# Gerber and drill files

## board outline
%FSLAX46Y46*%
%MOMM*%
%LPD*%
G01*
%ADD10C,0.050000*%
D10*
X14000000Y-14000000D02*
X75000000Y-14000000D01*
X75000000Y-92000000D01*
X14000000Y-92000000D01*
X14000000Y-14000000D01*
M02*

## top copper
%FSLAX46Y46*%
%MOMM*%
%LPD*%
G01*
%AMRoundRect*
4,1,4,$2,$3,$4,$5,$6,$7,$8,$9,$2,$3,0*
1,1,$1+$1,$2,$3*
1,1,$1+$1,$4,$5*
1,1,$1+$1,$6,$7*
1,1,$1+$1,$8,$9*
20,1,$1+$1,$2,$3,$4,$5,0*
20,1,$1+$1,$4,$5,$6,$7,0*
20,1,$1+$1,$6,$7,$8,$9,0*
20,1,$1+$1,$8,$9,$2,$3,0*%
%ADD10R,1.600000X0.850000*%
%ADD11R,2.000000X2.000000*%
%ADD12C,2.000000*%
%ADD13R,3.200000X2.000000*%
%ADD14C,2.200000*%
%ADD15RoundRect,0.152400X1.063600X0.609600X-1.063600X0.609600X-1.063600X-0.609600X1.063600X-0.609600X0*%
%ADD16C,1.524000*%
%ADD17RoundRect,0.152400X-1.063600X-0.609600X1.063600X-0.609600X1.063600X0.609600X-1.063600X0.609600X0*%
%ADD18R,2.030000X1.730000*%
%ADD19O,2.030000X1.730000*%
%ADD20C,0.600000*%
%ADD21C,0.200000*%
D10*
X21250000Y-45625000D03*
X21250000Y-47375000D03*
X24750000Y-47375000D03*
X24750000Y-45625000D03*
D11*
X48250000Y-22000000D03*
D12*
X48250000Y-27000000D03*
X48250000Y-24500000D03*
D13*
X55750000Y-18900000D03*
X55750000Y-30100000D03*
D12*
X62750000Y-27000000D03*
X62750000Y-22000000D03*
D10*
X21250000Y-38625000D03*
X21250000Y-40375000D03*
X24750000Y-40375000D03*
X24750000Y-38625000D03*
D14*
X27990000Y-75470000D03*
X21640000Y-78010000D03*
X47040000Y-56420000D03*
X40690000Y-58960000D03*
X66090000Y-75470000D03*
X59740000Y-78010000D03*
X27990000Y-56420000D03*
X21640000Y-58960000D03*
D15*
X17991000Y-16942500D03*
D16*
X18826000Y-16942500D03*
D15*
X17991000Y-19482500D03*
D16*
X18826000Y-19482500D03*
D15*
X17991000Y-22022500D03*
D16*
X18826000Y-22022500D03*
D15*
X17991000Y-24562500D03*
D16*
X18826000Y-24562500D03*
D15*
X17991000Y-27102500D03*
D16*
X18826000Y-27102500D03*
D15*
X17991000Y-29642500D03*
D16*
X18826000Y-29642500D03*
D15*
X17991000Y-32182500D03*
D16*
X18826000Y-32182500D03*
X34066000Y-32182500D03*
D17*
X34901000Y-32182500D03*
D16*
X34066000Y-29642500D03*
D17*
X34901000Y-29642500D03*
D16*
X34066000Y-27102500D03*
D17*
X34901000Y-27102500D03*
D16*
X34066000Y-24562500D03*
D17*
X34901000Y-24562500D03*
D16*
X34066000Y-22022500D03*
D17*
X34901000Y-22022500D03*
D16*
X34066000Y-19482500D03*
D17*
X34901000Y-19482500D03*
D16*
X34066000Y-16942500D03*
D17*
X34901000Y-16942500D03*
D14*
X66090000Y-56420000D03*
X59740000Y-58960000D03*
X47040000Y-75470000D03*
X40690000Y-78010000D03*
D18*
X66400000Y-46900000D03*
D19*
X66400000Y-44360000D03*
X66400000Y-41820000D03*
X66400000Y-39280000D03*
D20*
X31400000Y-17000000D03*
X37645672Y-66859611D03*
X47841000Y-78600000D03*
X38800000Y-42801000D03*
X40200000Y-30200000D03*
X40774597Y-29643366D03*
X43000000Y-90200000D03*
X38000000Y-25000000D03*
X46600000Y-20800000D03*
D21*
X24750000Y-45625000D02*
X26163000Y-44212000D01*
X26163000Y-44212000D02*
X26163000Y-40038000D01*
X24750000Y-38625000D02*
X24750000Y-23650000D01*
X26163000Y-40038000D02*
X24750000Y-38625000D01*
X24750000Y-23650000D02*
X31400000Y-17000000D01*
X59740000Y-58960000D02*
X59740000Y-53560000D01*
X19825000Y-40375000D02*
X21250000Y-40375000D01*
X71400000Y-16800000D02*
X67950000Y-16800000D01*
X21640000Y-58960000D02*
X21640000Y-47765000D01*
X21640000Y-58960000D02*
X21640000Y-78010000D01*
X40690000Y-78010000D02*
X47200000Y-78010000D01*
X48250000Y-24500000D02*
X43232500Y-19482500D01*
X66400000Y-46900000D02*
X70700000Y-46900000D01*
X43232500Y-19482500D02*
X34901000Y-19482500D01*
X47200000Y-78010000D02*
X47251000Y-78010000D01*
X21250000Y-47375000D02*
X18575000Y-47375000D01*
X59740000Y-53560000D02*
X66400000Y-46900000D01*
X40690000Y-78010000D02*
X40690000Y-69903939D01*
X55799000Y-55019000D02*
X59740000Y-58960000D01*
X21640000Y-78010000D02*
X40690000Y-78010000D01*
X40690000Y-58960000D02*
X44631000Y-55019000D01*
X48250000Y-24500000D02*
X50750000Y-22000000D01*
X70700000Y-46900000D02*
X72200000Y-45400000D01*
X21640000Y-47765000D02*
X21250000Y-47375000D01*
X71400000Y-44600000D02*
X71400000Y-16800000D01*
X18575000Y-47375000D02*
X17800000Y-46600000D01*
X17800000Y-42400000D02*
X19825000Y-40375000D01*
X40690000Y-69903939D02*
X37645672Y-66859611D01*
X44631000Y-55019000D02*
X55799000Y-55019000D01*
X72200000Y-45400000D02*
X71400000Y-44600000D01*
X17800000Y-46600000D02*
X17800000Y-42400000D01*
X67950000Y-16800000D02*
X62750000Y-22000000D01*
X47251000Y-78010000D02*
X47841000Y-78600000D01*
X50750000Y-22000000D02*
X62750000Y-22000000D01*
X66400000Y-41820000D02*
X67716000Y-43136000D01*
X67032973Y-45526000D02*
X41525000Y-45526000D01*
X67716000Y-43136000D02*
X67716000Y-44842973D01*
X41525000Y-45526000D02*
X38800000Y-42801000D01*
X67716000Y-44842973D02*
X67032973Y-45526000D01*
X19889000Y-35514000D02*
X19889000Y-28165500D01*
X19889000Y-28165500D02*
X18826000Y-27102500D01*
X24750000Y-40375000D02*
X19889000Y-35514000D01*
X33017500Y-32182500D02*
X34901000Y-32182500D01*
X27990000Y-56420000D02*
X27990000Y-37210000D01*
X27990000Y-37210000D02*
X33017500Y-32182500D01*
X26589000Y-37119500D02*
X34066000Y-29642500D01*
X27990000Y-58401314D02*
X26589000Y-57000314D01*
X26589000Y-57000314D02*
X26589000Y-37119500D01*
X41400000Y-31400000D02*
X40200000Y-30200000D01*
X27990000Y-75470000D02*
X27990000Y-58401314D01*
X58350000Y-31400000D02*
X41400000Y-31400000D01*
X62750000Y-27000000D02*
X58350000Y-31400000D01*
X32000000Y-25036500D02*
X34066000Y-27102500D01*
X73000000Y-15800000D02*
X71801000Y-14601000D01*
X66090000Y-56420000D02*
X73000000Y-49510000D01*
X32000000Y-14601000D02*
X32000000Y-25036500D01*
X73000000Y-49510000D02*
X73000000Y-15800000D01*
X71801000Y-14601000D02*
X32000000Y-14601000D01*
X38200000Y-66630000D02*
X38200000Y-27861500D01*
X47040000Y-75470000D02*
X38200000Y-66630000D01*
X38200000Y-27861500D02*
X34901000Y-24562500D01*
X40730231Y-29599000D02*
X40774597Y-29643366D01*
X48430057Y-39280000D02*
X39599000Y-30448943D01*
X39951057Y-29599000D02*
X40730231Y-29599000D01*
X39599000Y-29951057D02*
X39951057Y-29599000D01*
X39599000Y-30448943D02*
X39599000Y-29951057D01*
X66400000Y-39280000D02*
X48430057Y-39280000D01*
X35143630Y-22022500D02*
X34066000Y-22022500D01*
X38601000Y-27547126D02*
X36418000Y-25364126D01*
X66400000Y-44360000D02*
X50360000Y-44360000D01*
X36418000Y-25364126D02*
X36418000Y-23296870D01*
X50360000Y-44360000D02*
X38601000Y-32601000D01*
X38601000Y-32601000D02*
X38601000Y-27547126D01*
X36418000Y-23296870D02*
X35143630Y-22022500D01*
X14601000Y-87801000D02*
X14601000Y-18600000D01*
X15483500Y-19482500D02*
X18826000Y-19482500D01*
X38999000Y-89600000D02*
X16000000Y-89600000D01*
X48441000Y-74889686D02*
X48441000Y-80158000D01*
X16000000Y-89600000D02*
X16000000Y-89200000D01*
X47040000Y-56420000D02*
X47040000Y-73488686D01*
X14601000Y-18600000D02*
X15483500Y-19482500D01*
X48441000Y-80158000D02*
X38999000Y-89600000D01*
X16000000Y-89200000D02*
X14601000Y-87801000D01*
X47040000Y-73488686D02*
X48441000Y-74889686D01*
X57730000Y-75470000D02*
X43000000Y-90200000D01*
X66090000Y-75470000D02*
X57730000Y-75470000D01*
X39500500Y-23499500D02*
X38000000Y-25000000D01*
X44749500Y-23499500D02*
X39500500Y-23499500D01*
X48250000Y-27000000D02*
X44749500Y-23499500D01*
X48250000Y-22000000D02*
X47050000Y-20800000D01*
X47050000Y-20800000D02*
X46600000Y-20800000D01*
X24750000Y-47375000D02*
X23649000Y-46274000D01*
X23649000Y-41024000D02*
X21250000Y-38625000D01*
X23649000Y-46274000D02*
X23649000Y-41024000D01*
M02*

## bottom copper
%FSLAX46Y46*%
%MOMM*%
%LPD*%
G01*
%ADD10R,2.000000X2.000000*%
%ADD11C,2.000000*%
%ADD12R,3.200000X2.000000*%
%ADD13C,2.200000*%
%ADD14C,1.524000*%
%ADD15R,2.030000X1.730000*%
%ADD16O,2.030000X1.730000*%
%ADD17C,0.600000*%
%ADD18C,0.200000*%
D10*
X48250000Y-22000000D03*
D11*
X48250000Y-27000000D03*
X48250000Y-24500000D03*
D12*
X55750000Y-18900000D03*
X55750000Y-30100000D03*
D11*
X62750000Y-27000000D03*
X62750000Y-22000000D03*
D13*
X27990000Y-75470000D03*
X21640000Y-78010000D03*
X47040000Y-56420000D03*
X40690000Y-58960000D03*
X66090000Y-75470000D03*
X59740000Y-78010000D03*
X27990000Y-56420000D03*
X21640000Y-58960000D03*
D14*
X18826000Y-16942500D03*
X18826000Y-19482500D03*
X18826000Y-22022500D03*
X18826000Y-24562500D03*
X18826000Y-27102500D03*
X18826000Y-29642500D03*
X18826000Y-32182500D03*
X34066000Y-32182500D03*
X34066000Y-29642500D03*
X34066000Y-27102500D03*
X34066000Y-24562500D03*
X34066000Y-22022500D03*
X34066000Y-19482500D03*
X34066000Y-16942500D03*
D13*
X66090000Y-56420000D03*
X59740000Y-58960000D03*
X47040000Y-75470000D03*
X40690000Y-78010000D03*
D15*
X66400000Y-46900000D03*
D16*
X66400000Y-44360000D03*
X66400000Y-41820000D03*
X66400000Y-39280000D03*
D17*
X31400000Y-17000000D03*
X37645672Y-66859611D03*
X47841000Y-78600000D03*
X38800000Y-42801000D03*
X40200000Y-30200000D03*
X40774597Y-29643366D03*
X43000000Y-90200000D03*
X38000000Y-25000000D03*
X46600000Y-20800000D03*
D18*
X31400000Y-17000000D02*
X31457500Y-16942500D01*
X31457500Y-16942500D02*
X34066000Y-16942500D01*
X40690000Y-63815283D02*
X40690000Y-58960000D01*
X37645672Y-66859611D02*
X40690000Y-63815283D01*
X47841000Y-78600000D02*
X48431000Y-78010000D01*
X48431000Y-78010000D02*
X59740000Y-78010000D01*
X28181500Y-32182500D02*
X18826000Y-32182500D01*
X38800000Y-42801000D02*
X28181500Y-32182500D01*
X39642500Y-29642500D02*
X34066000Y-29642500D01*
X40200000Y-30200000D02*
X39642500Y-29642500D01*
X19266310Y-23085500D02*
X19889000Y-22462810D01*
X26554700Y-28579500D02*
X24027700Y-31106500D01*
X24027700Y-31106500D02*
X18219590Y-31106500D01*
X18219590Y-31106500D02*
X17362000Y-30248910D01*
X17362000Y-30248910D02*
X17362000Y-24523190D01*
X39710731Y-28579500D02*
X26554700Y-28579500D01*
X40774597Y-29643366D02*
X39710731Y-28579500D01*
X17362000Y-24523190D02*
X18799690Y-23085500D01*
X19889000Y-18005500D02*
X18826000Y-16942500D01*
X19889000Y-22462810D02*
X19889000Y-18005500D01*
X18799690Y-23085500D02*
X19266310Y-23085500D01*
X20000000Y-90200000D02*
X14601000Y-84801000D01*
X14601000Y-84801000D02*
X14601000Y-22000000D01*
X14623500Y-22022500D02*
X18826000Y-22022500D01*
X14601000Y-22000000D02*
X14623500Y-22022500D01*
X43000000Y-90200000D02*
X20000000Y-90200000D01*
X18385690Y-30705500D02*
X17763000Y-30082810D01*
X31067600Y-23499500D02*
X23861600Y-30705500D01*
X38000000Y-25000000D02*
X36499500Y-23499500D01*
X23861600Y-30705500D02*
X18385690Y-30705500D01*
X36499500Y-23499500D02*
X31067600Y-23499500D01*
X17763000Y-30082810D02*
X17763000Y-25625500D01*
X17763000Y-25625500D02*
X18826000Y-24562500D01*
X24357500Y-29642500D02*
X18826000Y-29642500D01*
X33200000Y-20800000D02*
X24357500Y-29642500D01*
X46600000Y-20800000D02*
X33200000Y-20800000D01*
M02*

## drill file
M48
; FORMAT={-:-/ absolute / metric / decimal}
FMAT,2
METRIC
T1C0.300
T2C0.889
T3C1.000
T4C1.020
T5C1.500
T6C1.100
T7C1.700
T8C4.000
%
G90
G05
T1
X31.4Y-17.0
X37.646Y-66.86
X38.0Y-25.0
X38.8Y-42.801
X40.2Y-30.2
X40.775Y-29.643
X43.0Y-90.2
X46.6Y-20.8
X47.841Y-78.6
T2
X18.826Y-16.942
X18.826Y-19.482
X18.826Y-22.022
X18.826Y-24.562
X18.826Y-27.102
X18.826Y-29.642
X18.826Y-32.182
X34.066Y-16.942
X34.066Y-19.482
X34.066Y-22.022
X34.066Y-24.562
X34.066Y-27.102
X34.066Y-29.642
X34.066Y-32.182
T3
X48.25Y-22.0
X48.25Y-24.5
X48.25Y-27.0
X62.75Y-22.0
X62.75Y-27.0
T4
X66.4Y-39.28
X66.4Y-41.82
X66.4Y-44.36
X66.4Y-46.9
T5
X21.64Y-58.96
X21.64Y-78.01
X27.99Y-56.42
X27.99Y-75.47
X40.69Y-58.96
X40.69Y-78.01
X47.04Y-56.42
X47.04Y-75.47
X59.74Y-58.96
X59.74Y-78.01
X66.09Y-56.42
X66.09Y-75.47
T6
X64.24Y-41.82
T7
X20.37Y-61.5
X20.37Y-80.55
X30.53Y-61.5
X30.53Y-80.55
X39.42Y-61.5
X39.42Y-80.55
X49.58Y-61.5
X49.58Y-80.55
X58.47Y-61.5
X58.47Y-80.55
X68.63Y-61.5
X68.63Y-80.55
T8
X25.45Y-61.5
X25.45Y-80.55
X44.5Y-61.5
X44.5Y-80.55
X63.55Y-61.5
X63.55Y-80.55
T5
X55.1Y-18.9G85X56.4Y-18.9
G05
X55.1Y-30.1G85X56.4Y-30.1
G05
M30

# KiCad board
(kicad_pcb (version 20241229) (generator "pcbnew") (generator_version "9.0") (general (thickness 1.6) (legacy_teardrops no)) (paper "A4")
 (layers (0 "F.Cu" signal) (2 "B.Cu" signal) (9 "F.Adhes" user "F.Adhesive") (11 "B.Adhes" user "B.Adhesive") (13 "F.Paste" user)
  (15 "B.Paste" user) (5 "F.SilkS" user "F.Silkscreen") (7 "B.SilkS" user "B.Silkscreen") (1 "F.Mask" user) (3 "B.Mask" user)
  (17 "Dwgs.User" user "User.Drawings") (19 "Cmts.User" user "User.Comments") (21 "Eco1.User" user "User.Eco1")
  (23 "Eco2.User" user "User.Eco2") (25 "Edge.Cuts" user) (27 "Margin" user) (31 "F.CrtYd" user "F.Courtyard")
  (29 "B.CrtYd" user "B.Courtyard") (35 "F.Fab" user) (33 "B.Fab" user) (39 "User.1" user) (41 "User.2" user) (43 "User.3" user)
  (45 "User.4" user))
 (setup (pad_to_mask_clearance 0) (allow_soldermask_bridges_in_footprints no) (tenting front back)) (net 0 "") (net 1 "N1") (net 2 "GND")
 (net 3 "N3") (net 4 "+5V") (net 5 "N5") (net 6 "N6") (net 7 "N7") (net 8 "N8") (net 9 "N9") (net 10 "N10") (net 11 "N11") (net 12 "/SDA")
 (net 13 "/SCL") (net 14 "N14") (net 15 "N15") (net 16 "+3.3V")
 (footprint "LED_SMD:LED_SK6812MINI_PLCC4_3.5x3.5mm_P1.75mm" (layer "F.Cu") (at 23 46.5)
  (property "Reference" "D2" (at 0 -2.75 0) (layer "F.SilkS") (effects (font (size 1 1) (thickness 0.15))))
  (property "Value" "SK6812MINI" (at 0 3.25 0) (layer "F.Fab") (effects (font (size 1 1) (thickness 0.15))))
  (pad "1" smd rect (at -1.75 -0.875) (size 1.6 0.85) (layers "F.Cu" "F.Mask" "F.Paste") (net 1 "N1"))
  (pad "2" smd rect (at -1.75 0.875) (size 1.6 0.85) (layers "F.Cu" "F.Mask" "F.Paste") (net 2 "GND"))
  (pad "3" smd rect (at 1.75 0.875) (size 1.6 0.85) (layers "F.Cu" "F.Mask" "F.Paste") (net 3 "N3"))
  (pad "4" smd rect (at 1.75 -0.875) (size 1.6 0.85) (layers "F.Cu" "F.Mask" "F.Paste") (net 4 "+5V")))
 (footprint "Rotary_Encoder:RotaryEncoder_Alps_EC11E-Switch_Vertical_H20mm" (layer "F.Cu") (at 48.25 22)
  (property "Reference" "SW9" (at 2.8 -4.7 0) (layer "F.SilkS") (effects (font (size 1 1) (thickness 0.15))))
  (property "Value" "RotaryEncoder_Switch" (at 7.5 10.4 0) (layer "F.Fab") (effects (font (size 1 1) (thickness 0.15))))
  (pad "A" thru_hole rect (at 0 0) (size 2 2) (drill 1) (layers "*.Cu" "*.Mask") (remove_unused_layers no) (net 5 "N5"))
  (pad "B" thru_hole circle (at 0 5) (size 2 2) (drill 1) (layers "*.Cu" "*.Mask") (remove_unused_layers no) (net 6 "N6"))
  (pad "C" thru_hole circle (at 0 2.5) (size 2 2) (drill 1) (layers "*.Cu" "*.Mask") (remove_unused_layers no) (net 2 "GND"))
  (pad "MP" thru_hole rect (at 7.5 -3.1) (size 3.2 2) (drill oval 2.8 1.5) (layers "*.Cu" "*.Mask") (remove_unused_layers no))
  (pad "MP" thru_hole rect (at 7.5 8.1) (size 3.2 2) (drill oval 2.8 1.5) (layers "*.Cu" "*.Mask") (remove_unused_layers no))
  (pad "S1" thru_hole circle (at 14.5 5) (size 2 2) (drill 1) (layers "*.Cu" "*.Mask") (remove_unused_layers no) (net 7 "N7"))
  (pad "S2" thru_hole circle (at 14.5 0) (size 2 2) (drill 1) (layers "*.Cu" "*.Mask") (remove_unused_layers no) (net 2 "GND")))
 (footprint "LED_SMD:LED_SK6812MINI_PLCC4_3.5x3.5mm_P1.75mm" (layer "F.Cu") (at 23 39.5)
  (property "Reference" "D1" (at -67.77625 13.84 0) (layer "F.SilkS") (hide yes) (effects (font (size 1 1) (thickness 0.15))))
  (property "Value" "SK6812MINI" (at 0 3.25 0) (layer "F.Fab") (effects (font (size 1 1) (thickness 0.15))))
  (pad "1" smd rect (at -1.75 -0.875) (size 1.6 0.85) (layers "F.Cu" "F.Mask" "F.Paste") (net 3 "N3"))
  (pad "2" smd rect (at -1.75 0.875) (size 1.6 0.85) (layers "F.Cu" "F.Mask" "F.Paste") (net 2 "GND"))
  (pad "3" smd rect (at 1.75 0.875) (size 1.6 0.85) (layers "F.Cu" "F.Mask" "F.Paste") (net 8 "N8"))
  (pad "4" smd rect (at 1.75 -0.875) (size 1.6 0.85) (layers "F.Cu" "F.Mask" "F.Paste") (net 4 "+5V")))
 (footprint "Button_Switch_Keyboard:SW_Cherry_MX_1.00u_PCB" (layer "F.Cu") (at 27.99 75.47)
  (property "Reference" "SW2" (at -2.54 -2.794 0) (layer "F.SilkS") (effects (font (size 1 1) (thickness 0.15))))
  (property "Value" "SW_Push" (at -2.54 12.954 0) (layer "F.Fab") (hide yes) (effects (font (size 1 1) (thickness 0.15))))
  (pad "" np_thru_hole circle (at -7.62 5.08) (size 1.7 1.7) (drill 1.7) (layers "*.Cu" "*.Mask"))
  (pad "" np_thru_hole circle (at -2.54 5.08) (size 4 4) (drill 4) (layers "*.Cu" "*.Mask"))
  (pad "" np_thru_hole circle (at 2.54 5.08) (size 1.7 1.7) (drill 1.7) (layers "*.Cu" "*.Mask"))
  (pad "1" thru_hole circle (at 0 0) (size 2.2 2.2) (drill 1.5) (layers "*.Cu" "*.Mask") (remove_unused_layers no) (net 7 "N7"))
  (pad "2" thru_hole circle (at -6.35 2.54) (size 2.2 2.2) (drill 1.5) (layers "*.Cu" "*.Mask") (remove_unused_layers no) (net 2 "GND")))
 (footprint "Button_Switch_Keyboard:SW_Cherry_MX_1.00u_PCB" (layer "F.Cu") (at 47.04 56.42)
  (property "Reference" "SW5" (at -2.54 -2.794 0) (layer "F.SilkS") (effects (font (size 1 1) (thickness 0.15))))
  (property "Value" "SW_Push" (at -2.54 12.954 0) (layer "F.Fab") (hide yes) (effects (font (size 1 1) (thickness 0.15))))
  (pad "" np_thru_hole circle (at -7.62 5.08) (size 1.7 1.7) (drill 1.7) (layers "*.Cu" "*.Mask"))
  (pad "" np_thru_hole circle (at -2.54 5.08) (size 4 4) (drill 4) (layers "*.Cu" "*.Mask"))
  (pad "" np_thru_hole circle (at 2.54 5.08) (size 1.7 1.7) (drill 1.7) (layers "*.Cu" "*.Mask"))
  (pad "1" thru_hole circle (at 0 0) (size 2.2 2.2) (drill 1.5) (layers "*.Cu" "*.Mask") (remove_unused_layers no) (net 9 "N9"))
  (pad "2" thru_hole circle (at -6.35 2.54) (size 2.2 2.2) (drill 1.5) (layers "*.Cu" "*.Mask") (remove_unused_layers no) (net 2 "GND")))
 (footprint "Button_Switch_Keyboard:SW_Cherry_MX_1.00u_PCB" (layer "F.Cu") (at 66.09 75.47)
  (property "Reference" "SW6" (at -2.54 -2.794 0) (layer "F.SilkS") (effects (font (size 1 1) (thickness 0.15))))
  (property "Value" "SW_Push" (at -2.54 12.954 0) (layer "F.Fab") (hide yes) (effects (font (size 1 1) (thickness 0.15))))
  (pad "" np_thru_hole circle (at -7.62 5.08) (size 1.7 1.7) (drill 1.7) (layers "*.Cu" "*.Mask"))
  (pad "" np_thru_hole circle (at -2.54 5.08) (size 4 4) (drill 4) (layers "*.Cu" "*.Mask"))
  (pad "" np_thru_hole circle (at 2.54 5.08) (size 1.7 1.7) (drill 1.7) (layers "*.Cu" "*.Mask"))
  (pad "1" thru_hole circle (at 0 0) (size 2.2 2.2) (drill 1.5) (layers "*.Cu" "*.Mask") (remove_unused_layers no) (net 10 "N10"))
  (pad "2" thru_hole circle (at -6.35 2.54) (size 2.2 2.2) (drill 1.5) (layers "*.Cu" "*.Mask") (remove_unused_layers no) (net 2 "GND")))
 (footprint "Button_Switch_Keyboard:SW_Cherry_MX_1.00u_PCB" (layer "F.Cu") (at 27.99 56.42)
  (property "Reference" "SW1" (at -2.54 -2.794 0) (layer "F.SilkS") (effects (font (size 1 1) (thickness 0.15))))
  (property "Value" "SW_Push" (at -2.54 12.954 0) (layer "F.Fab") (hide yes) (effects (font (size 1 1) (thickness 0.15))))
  (pad "" np_thru_hole circle (at -7.62 5.08) (size 1.7 1.7) (drill 1.7) (layers "*.Cu" "*.Mask"))
  (pad "" np_thru_hole circle (at -2.54 5.08) (size 4 4) (drill 4) (layers "*.Cu" "*.Mask"))
  (pad "" np_thru_hole circle (at 2.54 5.08) (size 1.7 1.7) (drill 1.7) (layers "*.Cu" "*.Mask"))
  (pad "1" thru_hole circle (at 0 0) (size 2.2 2.2) (drill 1.5) (layers "*.Cu" "*.Mask") (remove_unused_layers no) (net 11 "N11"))
  (pad "2" thru_hole circle (at -6.35 2.54) (size 2.2 2.2) (drill 1.5) (layers "*.Cu" "*.Mask") (remove_unused_layers no) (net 2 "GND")))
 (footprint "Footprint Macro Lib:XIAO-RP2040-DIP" (layer "F.Cu") (at 26.446 24.5625)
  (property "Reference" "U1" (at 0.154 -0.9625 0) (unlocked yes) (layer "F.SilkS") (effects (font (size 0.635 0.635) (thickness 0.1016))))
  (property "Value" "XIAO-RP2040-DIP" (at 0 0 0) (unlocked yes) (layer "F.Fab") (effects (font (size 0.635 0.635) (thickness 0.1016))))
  (pad "1" smd roundrect (at -8.455 -7.62 180) (size 2.432 1.524) (layers "F.Cu" "F.Mask") (roundrect_rratio 0.1) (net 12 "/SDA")
   (thermal_bridge_angle 45))
  (pad "1" thru_hole circle (at -7.62 -7.62 180) (size 1.524 1.524) (drill 0.889) (layers "*.Cu" "*.Mask") (remove_unused_layers no)
   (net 12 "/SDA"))
  (pad "2" smd roundrect (at -8.455 -5.08 180) (size 2.432 1.524) (layers "F.Cu" "F.Mask") (roundrect_rratio 0.1) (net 9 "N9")
   (thermal_bridge_angle 45))
  (pad "2" thru_hole circle (at -7.62 -5.08 180) (size 1.524 1.524) (drill 0.889) (layers "*.Cu" "*.Mask") (remove_unused_layers no)
   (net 9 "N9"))
  (pad "3" smd roundrect (at -8.455 -2.54 180) (size 2.432 1.524) (layers "F.Cu" "F.Mask") (roundrect_rratio 0.1) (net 10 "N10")
   (thermal_bridge_angle 45))
  (pad "3" thru_hole circle (at -7.62 -2.54 180) (size 1.524 1.524) (drill 0.889) (layers "*.Cu" "*.Mask") (remove_unused_layers no)
   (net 10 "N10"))
  (pad "4" smd roundrect (at -8.455 0 180) (size 2.432 1.524) (layers "F.Cu" "F.Mask") (roundrect_rratio 0.1) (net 6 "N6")
   (thermal_bridge_angle 45))
  (pad "4" thru_hole circle (at -7.62 0 180) (size 1.524 1.524) (drill 0.889) (layers "*.Cu" "*.Mask") (remove_unused_layers no)
   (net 6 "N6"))
  (pad "5" smd roundrect (at -8.455 2.54 180) (size 2.432 1.524) (layers "F.Cu" "F.Mask") (roundrect_rratio 0.1) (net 8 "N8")
   (thermal_bridge_angle 45))
  (pad "5" thru_hole circle (at -7.62 2.54 180) (size 1.524 1.524) (drill 0.889) (layers "*.Cu" "*.Mask") (remove_unused_layers no)
   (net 8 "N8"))
  (pad "6" smd roundrect (at -8.455 5.08 180) (size 2.432 1.524) (layers "F.Cu" "F.Mask") (roundrect_rratio 0.1) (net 5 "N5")
   (thermal_bridge_angle 45))
  (pad "6" thru_hole circle (at -7.62 5.08 180) (size 1.524 1.524) (drill 0.889) (layers "*.Cu" "*.Mask") (remove_unused_layers no)
   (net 5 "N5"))
  (pad "7" smd roundrect (at -8.455 7.62 180) (size 2.432 1.524) (layers "F.Cu" "F.Mask") (roundrect_rratio 0.1) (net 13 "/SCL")
   (thermal_bridge_angle 45))
  (pad "7" thru_hole circle (at -7.62 7.62 180) (size 1.524 1.524) (drill 0.889) (layers "*.Cu" "*.Mask") (remove_unused_layers no)
   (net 13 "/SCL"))
  (pad "8" thru_hole circle (at 7.62 7.62) (size 1.524 1.524) (drill 0.889) (layers "*.Cu" "*.Mask") (remove_unused_layers no)
   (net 11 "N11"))
  (pad "8" smd roundrect (at 8.455 7.62) (size 2.432 1.524) (layers "F.Cu" "F.Mask") (roundrect_rratio 0.1) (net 11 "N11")
   (thermal_bridge_angle 45))
  (pad "9" thru_hole circle (at 7.62 5.08) (size 1.524 1.524) (drill 0.889) (layers "*.Cu" "*.Mask") (remove_unused_layers no) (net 7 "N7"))
  (pad "9" smd roundrect (at 8.455 5.08) (size 2.432 1.524) (layers "F.Cu" "F.Mask") (roundrect_rratio 0.1) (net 7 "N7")
   (thermal_bridge_angle 45))
  (pad "10" thru_hole circle (at 7.62 2.54) (size 1.524 1.524) (drill 0.889) (layers "*.Cu" "*.Mask") (remove_unused_layers no)
   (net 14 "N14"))
  (pad "10" smd roundrect (at 8.455 2.54) (size 2.432 1.524) (layers "F.Cu" "F.Mask") (roundrect_rratio 0.1) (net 14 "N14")
   (thermal_bridge_angle 45))
  (pad "11" thru_hole circle (at 7.62 0) (size 1.524 1.524) (drill 0.889) (layers "*.Cu" "*.Mask") (remove_unused_layers no) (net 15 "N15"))
  (pad "11" smd roundrect (at 8.455 0) (size 2.432 1.524) (layers "F.Cu" "F.Mask") (roundrect_rratio 0.1) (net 15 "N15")
   (thermal_bridge_angle 45))
  (pad "12" thru_hole circle (at 7.62 -2.54) (size 1.524 1.524) (drill 0.889) (layers "*.Cu" "*.Mask") (remove_unused_layers no)
   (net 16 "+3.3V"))
  (pad "12" smd roundrect (at 8.455 -2.54) (size 2.432 1.524) (layers "F.Cu" "F.Mask") (roundrect_rratio 0.1) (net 16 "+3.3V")
   (thermal_bridge_angle 45))
  (pad "13" thru_hole circle (at 7.62 -5.08) (size 1.524 1.524) (drill 0.889) (layers "*.Cu" "*.Mask") (remove_unused_layers no)
   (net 2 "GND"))
  (pad "13" smd roundrect (at 8.455 -5.08) (size 2.432 1.524) (layers "F.Cu" "F.Mask") (roundrect_rratio 0.1) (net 2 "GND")
   (thermal_bridge_angle 45))
  (pad "14" thru_hole circle (at 7.62 -7.62) (size 1.524 1.524) (drill 0.889) (layers "*.Cu" "*.Mask") (remove_unused_layers no)
   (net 4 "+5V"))
  (pad "14" smd roundrect (at 8.455 -7.62) (size 2.432 1.524) (layers "F.Cu" "F.Mask") (roundrect_rratio 0.1) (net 4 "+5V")
   (thermal_bridge_angle 45)))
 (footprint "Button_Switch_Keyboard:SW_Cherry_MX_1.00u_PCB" (layer "F.Cu") (at 66.09 56.42)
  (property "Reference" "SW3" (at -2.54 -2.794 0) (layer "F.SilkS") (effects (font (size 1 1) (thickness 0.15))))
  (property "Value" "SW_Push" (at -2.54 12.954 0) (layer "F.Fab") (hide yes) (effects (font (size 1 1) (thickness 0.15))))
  (pad "" np_thru_hole circle (at -7.62 5.08) (size 1.7 1.7) (drill 1.7) (layers "*.Cu" "*.Mask"))
  (pad "" np_thru_hole circle (at -2.54 5.08) (size 4 4) (drill 4) (layers "*.Cu" "*.Mask"))
  (pad "" np_thru_hole circle (at 2.54 5.08) (size 1.7 1.7) (drill 1.7) (layers "*.Cu" "*.Mask"))
  (pad "1" thru_hole circle (at 0 0) (size 2.2 2.2) (drill 1.5) (layers "*.Cu" "*.Mask") (remove_unused_layers no) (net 14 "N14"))
  (pad "2" thru_hole circle (at -6.35 2.54) (size 2.2 2.2) (drill 1.5) (layers "*.Cu" "*.Mask") (remove_unused_layers no) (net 2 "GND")))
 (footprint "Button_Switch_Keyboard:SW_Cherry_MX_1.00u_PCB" (layer "F.Cu") (at 47.04 75.47)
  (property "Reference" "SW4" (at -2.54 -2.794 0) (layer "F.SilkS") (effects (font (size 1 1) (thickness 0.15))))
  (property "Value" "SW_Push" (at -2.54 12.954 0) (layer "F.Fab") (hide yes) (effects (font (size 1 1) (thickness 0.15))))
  (pad "" np_thru_hole circle (at -7.62 5.08) (size 1.7 1.7) (drill 1.7) (layers "*.Cu" "*.Mask"))
  (pad "" np_thru_hole circle (at -2.54 5.08) (size 4 4) (drill 4) (layers "*.Cu" "*.Mask"))
  (pad "" np_thru_hole circle (at 2.54 5.08) (size 1.7 1.7) (drill 1.7) (layers "*.Cu" "*.Mask"))
  (pad "1" thru_hole circle (at 0 0) (size 2.2 2.2) (drill 1.5) (layers "*.Cu" "*.Mask") (remove_unused_layers no) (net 15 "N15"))
  (pad "2" thru_hole circle (at -6.35 2.54) (size 2.2 2.2) (drill 1.5) (layers "*.Cu" "*.Mask") (remove_unused_layers no) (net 2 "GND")))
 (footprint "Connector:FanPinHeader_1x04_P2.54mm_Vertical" (layer "F.Cu") (at 66.4 46.9 90)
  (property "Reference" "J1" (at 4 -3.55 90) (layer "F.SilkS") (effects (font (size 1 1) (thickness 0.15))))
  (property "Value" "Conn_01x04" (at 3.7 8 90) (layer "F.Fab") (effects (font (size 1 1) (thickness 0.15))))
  (pad "" np_thru_hole circle (at 5.08 -2.16 180) (size 1.1 1.1) (drill 1.1) (layers "*.Cu" "*.Mask"))
  (pad "1" thru_hole rect (at 0 0 180) (size 2.03 1.73) (drill 1.02) (layers "*.Cu" "*.Mask") (remove_unused_layers no) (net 2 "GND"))
  (pad "2" thru_hole oval (at 2.54 0 180) (size 2.03 1.73) (drill 1.02) (layers "*.Cu" "*.Mask") (remove_unused_layers no) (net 16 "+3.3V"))
  (pad "3" thru_hole oval (at 5.08 0 180) (size 2.03 1.73) (drill 1.02) (layers "*.Cu" "*.Mask") (remove_unused_layers no) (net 13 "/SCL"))
  (pad "4" thru_hole oval (at 7.62 0 180) (size 2.03 1.73) (drill 1.02) (layers "*.Cu" "*.Mask") (remove_unused_layers no) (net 12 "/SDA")))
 (gr_rect (start 14 14) (end 75 92) (stroke (width 0.05) (type solid)) (fill no) (layer "Edge.Cuts"))
 (segment (start 24.75 45.625) (end 26.163 44.212) (width 0.2) (layer "F.Cu") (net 4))
 (segment (start 26.163 44.212) (end 26.163 40.038) (width 0.2) (layer "F.Cu") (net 4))
 (segment (start 24.75 38.625) (end 24.75 23.65) (width 0.2) (layer "F.Cu") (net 4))
 (segment (start 26.163 40.038) (end 24.75 38.625) (width 0.2) (layer "F.Cu") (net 4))
 (segment (start 24.75 23.65) (end 31.4 17) (width 0.2) (layer "F.Cu") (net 4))
 (via (at 31.4 17) (size 0.6) (drill 0.3) (layers "F.Cu" "B.Cu") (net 4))
 (segment (start 31.4 17) (end 31.4575 16.9425) (width 0.2) (layer "B.Cu") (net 4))
 (segment (start 31.4575 16.9425) (end 34.066 16.9425) (width 0.2) (layer "B.Cu") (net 4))
 (segment (start 59.74 58.96) (end 59.74 53.56) (width 0.2) (layer "F.Cu") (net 2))
 (segment (start 19.825 40.375) (end 21.25 40.375) (width 0.2) (layer "F.Cu") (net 2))
 (segment (start 71.4 16.8) (end 67.95 16.8) (width 0.2) (layer "F.Cu") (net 2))
 (segment (start 21.64 58.96) (end 21.64 47.765) (width 0.2) (layer "F.Cu") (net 2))
 (segment (start 21.64 58.96) (end 21.64 78.01) (width 0.2) (layer "F.Cu") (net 2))
 (segment (start 40.69 78.01) (end 47.2 78.01) (width 0.2) (layer "F.Cu") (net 2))
 (segment (start 48.25 24.5) (end 43.2325 19.4825) (width 0.2) (layer "F.Cu") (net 2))
 (segment (start 66.4 46.9) (end 70.7 46.9) (width 0.2) (layer "F.Cu") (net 2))
 (segment (start 43.2325 19.4825) (end 34.901 19.4825) (width 0.2) (layer "F.Cu") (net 2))
 (segment (start 47.2 78.01) (end 47.251 78.01) (width 0.2) (layer "F.Cu") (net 2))
 (segment (start 21.25 47.375) (end 18.575 47.375) (width 0.2) (layer "F.Cu") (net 2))
 (segment (start 59.74 53.56) (end 66.4 46.9) (width 0.2) (layer "F.Cu") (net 2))
 (segment (start 40.69 78.01) (end 40.69 69.903939) (width 0.2) (layer "F.Cu") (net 2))
 (segment (start 55.799 55.019) (end 59.74 58.96) (width 0.2) (layer "F.Cu") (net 2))
 (segment (start 21.64 78.01) (end 40.69 78.01) (width 0.2) (layer "F.Cu") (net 2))
 (segment (start 40.69 58.96) (end 44.631 55.019) (width 0.2) (layer "F.Cu") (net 2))
 (segment (start 48.25 24.5) (end 50.75 22) (width 0.2) (layer "F.Cu") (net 2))
 (segment (start 70.7 46.9) (end 72.2 45.4) (width 0.2) (layer "F.Cu") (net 2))
 (segment (start 21.64 47.765) (end 21.25 47.375) (width 0.2) (layer "F.Cu") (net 2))
 (segment (start 71.4 44.6) (end 71.4 16.8) (width 0.2) (layer "F.Cu") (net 2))
 (segment (start 18.575 47.375) (end 17.8 46.6) (width 0.2) (layer "F.Cu") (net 2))
 (segment (start 17.8 42.4) (end 19.825 40.375) (width 0.2) (layer "F.Cu") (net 2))
 (segment (start 40.69 69.903939) (end 37.645672 66.859611) (width 0.2) (layer "F.Cu") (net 2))
 (segment (start 44.631 55.019) (end 55.799 55.019) (width 0.2) (layer "F.Cu") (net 2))
 (segment (start 72.2 45.4) (end 71.4 44.6) (width 0.2) (layer "F.Cu") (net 2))
 (segment (start 17.8 46.6) (end 17.8 42.4) (width 0.2) (layer "F.Cu") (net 2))
 (segment (start 67.95 16.8) (end 62.75 22) (width 0.2) (layer "F.Cu") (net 2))
 (segment (start 47.251 78.01) (end 47.841 78.6) (width 0.2) (layer "F.Cu") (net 2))
 (segment (start 50.75 22) (end 62.75 22) (width 0.2) (layer "F.Cu") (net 2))
 (via (at 37.645672 66.859611) (size 0.6) (drill 0.3) (layers "F.Cu" "B.Cu") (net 2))
 (via (at 47.841 78.6) (size 0.6) (drill 0.3) (layers "F.Cu" "B.Cu") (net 2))
 (segment (start 40.69 63.815283) (end 40.69 58.96) (width 0.2) (layer "B.Cu") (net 2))
 (segment (start 37.645672 66.859611) (end 40.69 63.815283) (width 0.2) (layer "B.Cu") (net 2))
 (segment (start 47.841 78.6) (end 48.431 78.01) (width 0.2) (layer "B.Cu") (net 2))
 (segment (start 48.431 78.01) (end 59.74 78.01) (width 0.2) (layer "B.Cu") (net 2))
 (segment (start 66.4 41.82) (end 67.716 43.136) (width 0.2) (layer "F.Cu") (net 13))
 (segment (start 67.032973 45.526) (end 41.525 45.526) (width 0.2) (layer "F.Cu") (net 13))
 (segment (start 67.716 43.136) (end 67.716 44.842973) (width 0.2) (layer "F.Cu") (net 13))
 (segment (start 41.525 45.526) (end 38.8 42.801) (width 0.2) (layer "F.Cu") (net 13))
 (segment (start 67.716 44.842973) (end 67.032973 45.526) (width 0.2) (layer "F.Cu") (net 13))
 (via (at 38.8 42.801) (size 0.6) (drill 0.3) (layers "F.Cu" "B.Cu") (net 13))
 (segment (start 28.1815 32.1825) (end 18.826 32.1825) (width 0.2) (layer "B.Cu") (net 13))
 (segment (start 38.8 42.801) (end 28.1815 32.1825) (width 0.2) (layer "B.Cu") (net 13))
 (segment (start 19.889 35.514) (end 19.889 28.1655) (width 0.2) (layer "F.Cu") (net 8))
 (segment (start 19.889 28.1655) (end 18.826 27.1025) (width 0.2) (layer "F.Cu") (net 8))
 (segment (start 24.75 40.375) (end 19.889 35.514) (width 0.2) (layer "F.Cu") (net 8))
 (segment (start 33.0175 32.1825) (end 34.901 32.1825) (width 0.2) (layer "F.Cu") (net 11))
 (segment (start 27.99 56.42) (end 27.99 37.21) (width 0.2) (layer "F.Cu") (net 11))
 (segment (start 27.99 37.21) (end 33.0175 32.1825) (width 0.2) (layer "F.Cu") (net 11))
 (segment (start 26.589 37.1195) (end 34.066 29.6425) (width 0.2) (layer "F.Cu") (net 7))
 (segment (start 27.99 58.401314) (end 26.589 57.000314) (width 0.2) (layer "F.Cu") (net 7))
 (segment (start 26.589 57.000314) (end 26.589 37.1195) (width 0.2) (layer "F.Cu") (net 7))
 (segment (start 41.4 31.4) (end 40.2 30.2) (width 0.2) (layer "F.Cu") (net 7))
 (segment (start 27.99 75.47) (end 27.99 58.401314) (width 0.2) (layer "F.Cu") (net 7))
 (segment (start 58.35 31.4) (end 41.4 31.4) (width 0.2) (layer "F.Cu") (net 7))
 (segment (start 62.75 27) (end 58.35 31.4) (width 0.2) (layer "F.Cu") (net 7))
 (via (at 40.2 30.2) (size 0.6) (drill 0.3) (layers "F.Cu" "B.Cu") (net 7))
 (segment (start 39.6425 29.6425) (end 34.066 29.6425) (width 0.2) (layer "B.Cu") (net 7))
 (segment (start 40.2 30.2) (end 39.6425 29.6425) (width 0.2) (layer "B.Cu") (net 7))
 (segment (start 32 25.0365) (end 34.066 27.1025) (width 0.2) (layer "F.Cu") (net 14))
 (segment (start 73 15.8) (end 71.801 14.601) (width 0.2) (layer "F.Cu") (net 14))
 (segment (start 66.09 56.42) (end 73 49.51) (width 0.2) (layer "F.Cu") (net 14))
 (segment (start 32 14.601) (end 32 25.0365) (width 0.2) (layer "F.Cu") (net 14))
 (segment (start 73 49.51) (end 73 15.8) (width 0.2) (layer "F.Cu") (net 14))
 (segment (start 71.801 14.601) (end 32 14.601) (width 0.2) (layer "F.Cu") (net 14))
 (segment (start 38.2 66.63) (end 38.2 27.8615) (width 0.2) (layer "F.Cu") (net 15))
 (segment (start 47.04 75.47) (end 38.2 66.63) (width 0.2) (layer "F.Cu") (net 15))
 (segment (start 38.2 27.8615) (end 34.901 24.5625) (width 0.2) (layer "F.Cu") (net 15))
 (segment (start 40.730231 29.599) (end 40.774597 29.643366) (width 0.2) (layer "F.Cu") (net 12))
 (segment (start 48.430057 39.28) (end 39.599 30.448943) (width 0.2) (layer "F.Cu") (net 12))
 (segment (start 39.951057 29.599) (end 40.730231 29.599) (width 0.2) (layer "F.Cu") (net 12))
 (segment (start 39.599 29.951057) (end 39.951057 29.599) (width 0.2) (layer "F.Cu") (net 12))
 (segment (start 39.599 30.448943) (end 39.599 29.951057) (width 0.2) (layer "F.Cu") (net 12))
 (segment (start 66.4 39.28) (end 48.430057 39.28) (width 0.2) (layer "F.Cu") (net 12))
 (via (at 40.774597 29.643366) (size 0.6) (drill 0.3) (layers "F.Cu" "B.Cu") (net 12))
 (segment (start 19.26631 23.0855) (end 19.889 22.46281) (width 0.2) (layer "B.Cu") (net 12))
 (segment (start 26.5547 28.5795) (end 24.0277 31.1065) (width 0.2) (layer "B.Cu") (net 12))
 (segment (start 24.0277 31.1065) (end 18.21959 31.1065) (width 0.2) (layer "B.Cu") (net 12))
 (segment (start 18.21959 31.1065) (end 17.362 30.24891) (width 0.2) (layer "B.Cu") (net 12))
 (segment (start 17.362 30.24891) (end 17.362 24.52319) (width 0.2) (layer "B.Cu") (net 12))
 (segment (start 39.710731 28.5795) (end 26.5547 28.5795) (width 0.2) (layer "B.Cu") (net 12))
 (segment (start 40.774597 29.643366) (end 39.710731 28.5795) (width 0.2) (layer "B.Cu") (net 12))
 (segment (start 17.362 24.52319) (end 18.79969 23.0855) (width 0.2) (layer "B.Cu") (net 12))
 (segment (start 19.889 18.0055) (end 18.826 16.9425) (width 0.2) (layer "B.Cu") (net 12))
 (segment (start 19.889 22.46281) (end 19.889 18.0055) (width 0.2) (layer "B.Cu") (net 12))
 (segment (start 18.79969 23.0855) (end 19.26631 23.0855) (width 0.2) (layer "B.Cu") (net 12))
 (segment (start 35.14363 22.0225) (end 34.066 22.0225) (width 0.2) (layer "F.Cu") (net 16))
 (segment (start 38.601 27.547126) (end 36.418 25.364126) (width 0.2) (layer "F.Cu") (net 16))
 (segment (start 66.4 44.36) (end 50.36 44.36) (width 0.2) (layer "F.Cu") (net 16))
 (segment (start 36.418 25.364126) (end 36.418 23.29687) (width 0.2) (layer "F.Cu") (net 16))
 (segment (start 50.36 44.36) (end 38.601 32.601) (width 0.2) (layer "F.Cu") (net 16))
 (segment (start 38.601 32.601) (end 38.601 27.547126) (width 0.2) (layer "F.Cu") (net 16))
 (segment (start 36.418 23.29687) (end 35.14363 22.0225) (width 0.2) (layer "F.Cu") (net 16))
 (segment (start 14.601 87.801) (end 14.601 18.6) (width 0.2) (layer "F.Cu") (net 9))
 (segment (start 15.4835 19.4825) (end 18.826 19.4825) (width 0.2) (layer "F.Cu") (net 9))
 (segment (start 38.999 89.6) (end 16 89.6) (width 0.2) (layer "F.Cu") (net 9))
 (segment (start 48.441 74.889686) (end 48.441 80.158) (width 0.2) (layer "F.Cu") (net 9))
 (segment (start 16 89.6) (end 16 89.2) (width 0.2) (layer "F.Cu") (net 9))
 (segment (start 47.04 56.42) (end 47.04 73.488686) (width 0.2) (layer "F.Cu") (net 9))
 (segment (start 14.601 18.6) (end 15.4835 19.4825) (width 0.2) (layer "F.Cu") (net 9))
 (segment (start 48.441 80.158) (end 38.999 89.6) (width 0.2) (layer "F.Cu") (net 9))
 (segment (start 16 89.2) (end 14.601 87.801) (width 0.2) (layer "F.Cu") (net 9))
 (segment (start 47.04 73.488686) (end 48.441 74.889686) (width 0.2) (layer "F.Cu") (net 9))
 (segment (start 57.73 75.47) (end 43 90.2) (width 0.2) (layer "F.Cu") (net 10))
 (segment (start 66.09 75.47) (end 57.73 75.47) (width 0.2) (layer "F.Cu") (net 10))
 (via (at 43 90.2) (size 0.6) (drill 0.3) (layers "F.Cu" "B.Cu") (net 10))
 (segment (start 20 90.2) (end 14.601 84.801) (width 0.2) (layer "B.Cu") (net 10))
 (segment (start 14.601 84.801) (end 14.601 22) (width 0.2) (layer "B.Cu") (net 10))
 (segment (start 14.6235 22.0225) (end 18.826 22.0225) (width 0.2) (layer "B.Cu") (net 10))
 (segment (start 14.601 22) (end 14.6235 22.0225) (width 0.2) (layer "B.Cu") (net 10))
 (segment (start 43 90.2) (end 20 90.2) (width 0.2) (layer "B.Cu") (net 10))
 (segment (start 39.5005 23.4995) (end 38 25) (width 0.2) (layer "F.Cu") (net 6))
 (segment (start 44.7495 23.4995) (end 39.5005 23.4995) (width 0.2) (layer "F.Cu") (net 6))
 (segment (start 48.25 27) (end 44.7495 23.4995) (width 0.2) (layer "F.Cu") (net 6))
 (via (at 38 25) (size 0.6) (drill 0.3) (layers "F.Cu" "B.Cu") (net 6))
 (segment (start 18.38569 30.7055) (end 17.763 30.08281) (width 0.2) (layer "B.Cu") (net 6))
 (segment (start 31.0676 23.4995) (end 23.8616 30.7055) (width 0.2) (layer "B.Cu") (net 6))
 (segment (start 38 25) (end 36.4995 23.4995) (width 0.2) (layer "B.Cu") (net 6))
 (segment (start 23.8616 30.7055) (end 18.38569 30.7055) (width 0.2) (layer "B.Cu") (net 6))
 (segment (start 36.4995 23.4995) (end 31.0676 23.4995) (width 0.2) (layer "B.Cu") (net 6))
 (segment (start 17.763 30.08281) (end 17.763 25.6255) (width 0.2) (layer "B.Cu") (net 6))
 (segment (start 17.763 25.6255) (end 18.826 24.5625) (width 0.2) (layer "B.Cu") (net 6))
 (segment (start 48.25 22) (end 47.05 20.8) (width 0.2) (layer "F.Cu") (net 5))
 (segment (start 47.05 20.8) (end 46.6 20.8) (width 0.2) (layer "F.Cu") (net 5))
 (via (at 46.6 20.8) (size 0.6) (drill 0.3) (layers "F.Cu" "B.Cu") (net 5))
 (segment (start 24.3575 29.6425) (end 18.826 29.6425) (width 0.2) (layer "B.Cu") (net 5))
 (segment (start 33.2 20.8) (end 24.3575 29.6425) (width 0.2) (layer "B.Cu") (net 5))
 (segment (start 46.6 20.8) (end 33.2 20.8) (width 0.2) (layer "B.Cu") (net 5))
 (segment (start 24.75 47.375) (end 23.649 46.274) (width 0.2) (layer "F.Cu") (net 3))
 (segment (start 23.649 41.024) (end 21.25 38.625) (width 0.2) (layer "F.Cu") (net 3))
 (segment (start 23.649 46.274) (end 23.649 41.024) (width 0.2) (layer "F.Cu") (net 3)))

